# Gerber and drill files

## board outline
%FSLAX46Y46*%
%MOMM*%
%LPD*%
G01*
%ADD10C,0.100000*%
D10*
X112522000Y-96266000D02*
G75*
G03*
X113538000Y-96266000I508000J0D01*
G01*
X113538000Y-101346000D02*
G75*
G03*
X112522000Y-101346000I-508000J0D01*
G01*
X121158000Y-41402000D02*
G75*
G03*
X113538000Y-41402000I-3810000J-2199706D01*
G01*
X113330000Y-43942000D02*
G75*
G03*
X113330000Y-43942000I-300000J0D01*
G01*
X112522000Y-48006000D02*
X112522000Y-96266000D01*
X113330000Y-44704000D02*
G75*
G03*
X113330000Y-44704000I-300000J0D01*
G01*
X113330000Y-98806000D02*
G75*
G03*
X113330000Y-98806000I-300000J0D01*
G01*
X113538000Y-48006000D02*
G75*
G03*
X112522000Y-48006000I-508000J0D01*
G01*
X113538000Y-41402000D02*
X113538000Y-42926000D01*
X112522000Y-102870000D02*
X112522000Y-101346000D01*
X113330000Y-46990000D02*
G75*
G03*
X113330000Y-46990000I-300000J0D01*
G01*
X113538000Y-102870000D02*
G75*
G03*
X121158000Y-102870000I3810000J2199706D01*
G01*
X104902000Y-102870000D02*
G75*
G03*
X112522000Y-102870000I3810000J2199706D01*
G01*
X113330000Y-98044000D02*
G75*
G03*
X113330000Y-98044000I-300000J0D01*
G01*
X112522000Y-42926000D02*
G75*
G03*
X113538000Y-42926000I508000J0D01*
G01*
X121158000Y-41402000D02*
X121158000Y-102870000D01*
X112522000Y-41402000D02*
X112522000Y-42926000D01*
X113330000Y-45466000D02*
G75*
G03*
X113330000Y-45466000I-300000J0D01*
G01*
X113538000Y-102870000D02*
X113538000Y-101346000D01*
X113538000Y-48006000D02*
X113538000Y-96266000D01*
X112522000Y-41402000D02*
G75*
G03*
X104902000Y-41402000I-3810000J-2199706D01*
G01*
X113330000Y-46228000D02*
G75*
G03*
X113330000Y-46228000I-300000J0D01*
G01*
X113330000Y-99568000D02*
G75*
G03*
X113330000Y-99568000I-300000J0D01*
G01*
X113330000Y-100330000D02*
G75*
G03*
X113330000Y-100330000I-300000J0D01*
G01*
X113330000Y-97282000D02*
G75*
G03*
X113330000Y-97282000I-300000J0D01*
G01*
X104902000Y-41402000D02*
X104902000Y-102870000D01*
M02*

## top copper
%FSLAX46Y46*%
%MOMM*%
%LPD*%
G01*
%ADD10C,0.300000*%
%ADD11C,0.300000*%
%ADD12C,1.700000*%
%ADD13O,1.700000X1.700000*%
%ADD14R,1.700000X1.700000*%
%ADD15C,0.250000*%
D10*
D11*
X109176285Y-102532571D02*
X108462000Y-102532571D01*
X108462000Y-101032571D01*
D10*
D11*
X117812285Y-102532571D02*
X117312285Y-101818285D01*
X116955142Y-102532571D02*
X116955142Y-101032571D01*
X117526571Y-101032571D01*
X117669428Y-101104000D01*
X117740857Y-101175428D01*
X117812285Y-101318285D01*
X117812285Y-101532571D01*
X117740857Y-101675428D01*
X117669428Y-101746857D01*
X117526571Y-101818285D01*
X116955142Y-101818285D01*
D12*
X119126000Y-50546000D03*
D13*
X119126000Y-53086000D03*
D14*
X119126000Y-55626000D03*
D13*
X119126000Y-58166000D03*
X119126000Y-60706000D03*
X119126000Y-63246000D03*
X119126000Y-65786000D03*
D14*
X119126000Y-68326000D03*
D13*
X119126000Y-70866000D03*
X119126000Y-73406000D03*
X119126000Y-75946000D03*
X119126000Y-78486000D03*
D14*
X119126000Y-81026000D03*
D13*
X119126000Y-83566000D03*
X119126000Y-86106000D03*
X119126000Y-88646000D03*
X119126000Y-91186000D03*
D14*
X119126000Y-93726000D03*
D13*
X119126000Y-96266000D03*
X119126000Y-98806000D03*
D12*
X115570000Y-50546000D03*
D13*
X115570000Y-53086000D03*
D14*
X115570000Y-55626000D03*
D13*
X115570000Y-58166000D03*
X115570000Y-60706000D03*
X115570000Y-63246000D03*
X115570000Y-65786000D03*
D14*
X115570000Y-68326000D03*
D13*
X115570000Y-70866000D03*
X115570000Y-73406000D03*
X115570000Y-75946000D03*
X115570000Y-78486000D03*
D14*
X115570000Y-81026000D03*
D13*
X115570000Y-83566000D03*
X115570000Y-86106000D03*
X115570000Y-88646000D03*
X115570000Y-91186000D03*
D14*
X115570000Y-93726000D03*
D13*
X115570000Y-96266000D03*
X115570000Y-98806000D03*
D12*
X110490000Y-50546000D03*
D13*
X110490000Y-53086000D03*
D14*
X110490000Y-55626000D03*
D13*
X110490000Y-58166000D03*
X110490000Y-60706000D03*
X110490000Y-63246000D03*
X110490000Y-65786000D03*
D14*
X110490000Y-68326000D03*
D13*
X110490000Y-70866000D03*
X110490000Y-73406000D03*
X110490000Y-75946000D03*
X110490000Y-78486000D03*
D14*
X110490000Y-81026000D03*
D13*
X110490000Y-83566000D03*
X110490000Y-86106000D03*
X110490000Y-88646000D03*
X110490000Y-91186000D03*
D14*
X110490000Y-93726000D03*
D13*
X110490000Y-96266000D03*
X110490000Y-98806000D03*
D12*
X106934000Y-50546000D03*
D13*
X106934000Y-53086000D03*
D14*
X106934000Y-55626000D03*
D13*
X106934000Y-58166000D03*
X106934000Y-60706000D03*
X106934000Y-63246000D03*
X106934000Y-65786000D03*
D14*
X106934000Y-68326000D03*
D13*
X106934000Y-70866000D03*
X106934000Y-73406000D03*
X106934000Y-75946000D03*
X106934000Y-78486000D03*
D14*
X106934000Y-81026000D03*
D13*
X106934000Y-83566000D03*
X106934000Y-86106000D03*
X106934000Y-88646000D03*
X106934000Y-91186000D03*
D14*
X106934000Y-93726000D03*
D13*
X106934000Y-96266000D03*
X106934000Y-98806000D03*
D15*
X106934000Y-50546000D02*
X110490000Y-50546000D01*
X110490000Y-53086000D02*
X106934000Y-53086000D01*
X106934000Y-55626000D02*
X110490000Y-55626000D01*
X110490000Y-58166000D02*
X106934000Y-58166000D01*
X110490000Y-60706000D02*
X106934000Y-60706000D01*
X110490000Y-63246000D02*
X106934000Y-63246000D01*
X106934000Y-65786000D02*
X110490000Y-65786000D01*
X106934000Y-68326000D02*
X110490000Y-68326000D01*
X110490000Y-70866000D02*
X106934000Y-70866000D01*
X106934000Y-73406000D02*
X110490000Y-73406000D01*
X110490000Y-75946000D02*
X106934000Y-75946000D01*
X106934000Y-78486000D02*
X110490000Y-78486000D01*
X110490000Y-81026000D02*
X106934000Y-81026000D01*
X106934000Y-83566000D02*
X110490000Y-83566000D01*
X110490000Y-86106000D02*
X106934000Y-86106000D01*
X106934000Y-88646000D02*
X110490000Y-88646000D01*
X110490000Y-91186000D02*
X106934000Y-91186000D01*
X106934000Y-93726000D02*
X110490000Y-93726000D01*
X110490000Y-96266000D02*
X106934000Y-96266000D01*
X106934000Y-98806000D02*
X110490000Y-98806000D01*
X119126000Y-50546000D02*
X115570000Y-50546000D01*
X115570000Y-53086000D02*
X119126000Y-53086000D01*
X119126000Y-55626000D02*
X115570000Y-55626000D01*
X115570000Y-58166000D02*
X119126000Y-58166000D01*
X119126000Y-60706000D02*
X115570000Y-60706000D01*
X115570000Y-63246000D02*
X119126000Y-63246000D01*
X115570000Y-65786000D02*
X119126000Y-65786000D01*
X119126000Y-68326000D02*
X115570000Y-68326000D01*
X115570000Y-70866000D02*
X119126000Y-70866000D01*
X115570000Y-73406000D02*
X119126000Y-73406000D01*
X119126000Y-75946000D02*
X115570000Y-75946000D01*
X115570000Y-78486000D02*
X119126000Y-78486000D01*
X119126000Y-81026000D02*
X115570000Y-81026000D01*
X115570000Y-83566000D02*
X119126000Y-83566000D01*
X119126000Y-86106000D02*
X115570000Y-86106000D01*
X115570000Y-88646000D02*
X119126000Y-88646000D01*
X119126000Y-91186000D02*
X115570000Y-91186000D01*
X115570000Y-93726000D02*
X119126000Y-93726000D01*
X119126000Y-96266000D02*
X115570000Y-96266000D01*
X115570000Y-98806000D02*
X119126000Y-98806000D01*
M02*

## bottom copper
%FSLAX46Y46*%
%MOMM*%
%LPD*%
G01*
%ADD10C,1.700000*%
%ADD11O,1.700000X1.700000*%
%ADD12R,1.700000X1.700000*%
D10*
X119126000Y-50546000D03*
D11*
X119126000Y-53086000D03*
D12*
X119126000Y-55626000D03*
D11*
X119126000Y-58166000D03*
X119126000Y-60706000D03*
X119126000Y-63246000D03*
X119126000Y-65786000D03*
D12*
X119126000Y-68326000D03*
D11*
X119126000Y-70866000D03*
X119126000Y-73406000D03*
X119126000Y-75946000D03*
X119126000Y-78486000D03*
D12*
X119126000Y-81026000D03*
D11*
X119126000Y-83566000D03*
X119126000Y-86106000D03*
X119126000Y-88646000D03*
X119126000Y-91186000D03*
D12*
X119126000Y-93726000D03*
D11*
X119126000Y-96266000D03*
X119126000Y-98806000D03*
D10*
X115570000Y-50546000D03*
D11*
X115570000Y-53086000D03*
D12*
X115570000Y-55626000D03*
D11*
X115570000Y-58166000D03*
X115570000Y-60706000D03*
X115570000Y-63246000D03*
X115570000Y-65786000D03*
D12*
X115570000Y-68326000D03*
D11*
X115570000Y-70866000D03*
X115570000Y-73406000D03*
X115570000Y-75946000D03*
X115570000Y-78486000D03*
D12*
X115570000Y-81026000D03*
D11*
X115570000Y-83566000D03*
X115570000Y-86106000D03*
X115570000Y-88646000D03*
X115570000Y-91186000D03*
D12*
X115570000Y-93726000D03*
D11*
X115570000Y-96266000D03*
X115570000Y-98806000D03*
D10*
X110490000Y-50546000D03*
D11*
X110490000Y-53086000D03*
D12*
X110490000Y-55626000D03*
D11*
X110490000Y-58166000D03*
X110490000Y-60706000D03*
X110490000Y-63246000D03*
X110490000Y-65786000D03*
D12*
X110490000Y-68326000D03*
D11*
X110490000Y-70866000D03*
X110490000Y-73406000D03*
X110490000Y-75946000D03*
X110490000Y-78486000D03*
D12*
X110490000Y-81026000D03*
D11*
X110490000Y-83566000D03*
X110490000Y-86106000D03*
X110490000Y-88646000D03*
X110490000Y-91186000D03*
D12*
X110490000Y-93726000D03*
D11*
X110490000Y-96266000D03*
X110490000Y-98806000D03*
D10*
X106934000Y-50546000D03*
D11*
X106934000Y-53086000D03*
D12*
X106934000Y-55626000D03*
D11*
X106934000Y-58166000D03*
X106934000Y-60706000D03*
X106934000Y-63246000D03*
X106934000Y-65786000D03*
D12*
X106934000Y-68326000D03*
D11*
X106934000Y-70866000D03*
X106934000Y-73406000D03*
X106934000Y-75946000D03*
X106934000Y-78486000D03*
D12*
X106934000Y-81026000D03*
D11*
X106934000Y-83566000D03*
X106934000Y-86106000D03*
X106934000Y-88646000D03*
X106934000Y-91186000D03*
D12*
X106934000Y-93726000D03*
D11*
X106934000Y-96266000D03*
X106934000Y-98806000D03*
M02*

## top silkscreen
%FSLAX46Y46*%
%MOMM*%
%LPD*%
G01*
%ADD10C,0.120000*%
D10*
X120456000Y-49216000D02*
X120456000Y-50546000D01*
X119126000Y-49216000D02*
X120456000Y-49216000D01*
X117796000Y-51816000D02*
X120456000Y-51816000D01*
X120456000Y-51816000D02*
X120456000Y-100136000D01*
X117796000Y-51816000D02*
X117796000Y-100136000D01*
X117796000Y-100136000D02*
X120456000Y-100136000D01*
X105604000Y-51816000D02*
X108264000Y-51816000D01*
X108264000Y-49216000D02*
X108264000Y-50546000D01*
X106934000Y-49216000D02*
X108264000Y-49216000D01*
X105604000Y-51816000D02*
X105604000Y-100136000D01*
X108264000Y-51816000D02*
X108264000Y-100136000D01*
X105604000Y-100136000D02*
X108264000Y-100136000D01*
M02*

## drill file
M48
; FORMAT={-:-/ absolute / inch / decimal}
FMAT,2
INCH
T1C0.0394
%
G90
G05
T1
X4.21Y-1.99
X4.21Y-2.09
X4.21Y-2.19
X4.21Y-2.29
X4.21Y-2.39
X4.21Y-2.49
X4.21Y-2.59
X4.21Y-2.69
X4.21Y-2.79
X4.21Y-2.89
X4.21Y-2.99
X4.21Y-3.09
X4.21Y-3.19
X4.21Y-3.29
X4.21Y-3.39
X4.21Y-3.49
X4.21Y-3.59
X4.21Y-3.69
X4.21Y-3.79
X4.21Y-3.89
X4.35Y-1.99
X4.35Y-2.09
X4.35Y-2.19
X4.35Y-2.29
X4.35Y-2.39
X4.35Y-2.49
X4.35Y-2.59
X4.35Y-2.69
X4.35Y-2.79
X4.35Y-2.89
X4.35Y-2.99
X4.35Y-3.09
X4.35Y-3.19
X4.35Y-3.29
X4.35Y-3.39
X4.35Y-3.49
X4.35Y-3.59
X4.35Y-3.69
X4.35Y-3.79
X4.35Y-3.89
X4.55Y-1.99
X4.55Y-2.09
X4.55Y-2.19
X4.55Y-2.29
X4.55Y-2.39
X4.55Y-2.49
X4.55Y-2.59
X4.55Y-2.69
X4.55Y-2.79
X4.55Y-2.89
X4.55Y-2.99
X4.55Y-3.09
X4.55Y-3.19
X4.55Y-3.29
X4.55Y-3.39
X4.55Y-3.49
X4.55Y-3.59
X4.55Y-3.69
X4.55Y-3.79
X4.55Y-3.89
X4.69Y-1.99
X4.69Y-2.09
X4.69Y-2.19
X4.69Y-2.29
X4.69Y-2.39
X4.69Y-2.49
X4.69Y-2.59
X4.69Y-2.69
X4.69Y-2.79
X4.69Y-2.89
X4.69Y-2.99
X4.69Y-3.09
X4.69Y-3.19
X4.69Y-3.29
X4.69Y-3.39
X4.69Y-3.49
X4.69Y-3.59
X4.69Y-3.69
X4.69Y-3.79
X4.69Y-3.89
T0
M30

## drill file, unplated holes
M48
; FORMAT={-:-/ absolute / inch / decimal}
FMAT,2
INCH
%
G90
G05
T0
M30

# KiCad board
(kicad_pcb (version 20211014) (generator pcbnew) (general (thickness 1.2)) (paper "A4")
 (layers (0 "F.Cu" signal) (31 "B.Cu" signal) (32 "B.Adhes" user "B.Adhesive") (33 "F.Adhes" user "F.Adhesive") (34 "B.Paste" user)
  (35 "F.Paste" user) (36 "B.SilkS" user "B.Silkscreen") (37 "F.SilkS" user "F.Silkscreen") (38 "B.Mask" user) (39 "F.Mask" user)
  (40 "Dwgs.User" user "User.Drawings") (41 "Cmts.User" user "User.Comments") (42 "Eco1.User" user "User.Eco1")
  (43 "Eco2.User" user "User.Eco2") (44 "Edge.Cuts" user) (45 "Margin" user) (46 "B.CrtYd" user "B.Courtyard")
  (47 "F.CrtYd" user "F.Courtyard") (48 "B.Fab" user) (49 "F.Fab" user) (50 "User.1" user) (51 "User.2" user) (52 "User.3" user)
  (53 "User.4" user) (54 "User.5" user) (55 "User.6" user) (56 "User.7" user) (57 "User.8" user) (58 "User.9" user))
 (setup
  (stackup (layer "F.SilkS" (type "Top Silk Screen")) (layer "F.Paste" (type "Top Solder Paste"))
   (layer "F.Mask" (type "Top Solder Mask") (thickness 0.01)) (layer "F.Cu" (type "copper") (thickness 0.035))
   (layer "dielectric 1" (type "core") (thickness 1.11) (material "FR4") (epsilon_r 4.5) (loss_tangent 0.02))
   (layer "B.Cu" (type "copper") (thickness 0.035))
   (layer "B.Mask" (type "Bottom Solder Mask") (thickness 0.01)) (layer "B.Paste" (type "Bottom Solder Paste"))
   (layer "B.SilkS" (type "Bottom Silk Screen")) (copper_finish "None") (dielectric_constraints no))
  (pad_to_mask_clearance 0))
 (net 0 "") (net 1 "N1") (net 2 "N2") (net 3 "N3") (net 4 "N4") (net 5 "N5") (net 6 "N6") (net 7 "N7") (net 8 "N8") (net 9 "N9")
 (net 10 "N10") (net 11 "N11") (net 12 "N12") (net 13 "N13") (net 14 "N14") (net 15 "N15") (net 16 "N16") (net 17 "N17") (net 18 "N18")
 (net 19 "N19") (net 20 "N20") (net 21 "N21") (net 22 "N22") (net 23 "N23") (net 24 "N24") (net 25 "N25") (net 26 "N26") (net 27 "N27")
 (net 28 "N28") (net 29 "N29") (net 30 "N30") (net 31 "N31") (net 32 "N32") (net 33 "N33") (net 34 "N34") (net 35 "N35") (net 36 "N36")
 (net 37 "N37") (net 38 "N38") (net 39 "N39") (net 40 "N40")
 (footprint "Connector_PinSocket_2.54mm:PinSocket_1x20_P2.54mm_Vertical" (layer "F.Cu") (at 119.126 50.546)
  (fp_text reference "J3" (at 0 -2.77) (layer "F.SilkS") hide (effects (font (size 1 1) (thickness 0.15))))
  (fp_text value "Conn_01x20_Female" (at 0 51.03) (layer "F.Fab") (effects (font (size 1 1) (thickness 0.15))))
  (fp_line (start 1.33 -1.33) (end 1.33 0) (layer "F.SilkS") (width 0.12))
  (fp_line (start 0 -1.33) (end 1.33 -1.33) (layer "F.SilkS") (width 0.12))
  (fp_line (start -1.33 1.27) (end 1.33 1.27) (layer "F.SilkS") (width 0.12))
  (fp_line (start 1.33 1.27) (end 1.33 49.59) (layer "F.SilkS") (width 0.12))
  (fp_line (start -1.33 1.27) (end -1.33 49.59) (layer "F.SilkS") (width 0.12))
  (fp_line (start -1.33 49.59) (end 1.33 49.59) (layer "F.SilkS") (width 0.12))
  (pad "1" thru_hole circle (at 0 0) (size 1.7 1.7) (drill 1) (layers *.Cu *.Mask) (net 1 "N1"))
  (pad "2" thru_hole oval (at 0 2.54) (size 1.7 1.7) (drill 1) (layers *.Cu *.Mask) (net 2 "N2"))
  (pad "3" thru_hole rect (at 0 5.08) (size 1.7 1.7) (drill 1) (layers *.Cu *.Mask) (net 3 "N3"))
  (pad "4" thru_hole oval (at 0 7.62) (size 1.7 1.7) (drill 1) (layers *.Cu *.Mask) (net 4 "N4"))
  (pad "5" thru_hole oval (at 0 10.16) (size 1.7 1.7) (drill 1) (layers *.Cu *.Mask) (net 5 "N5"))
  (pad "6" thru_hole oval (at 0 12.7) (size 1.7 1.7) (drill 1) (layers *.Cu *.Mask) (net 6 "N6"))
  (pad "7" thru_hole oval (at 0 15.24) (size 1.7 1.7) (drill 1) (layers *.Cu *.Mask) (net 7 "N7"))
  (pad "8" thru_hole rect (at 0 17.78) (size 1.7 1.7) (drill 1) (layers *.Cu *.Mask) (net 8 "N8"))
  (pad "9" thru_hole oval (at 0 20.32) (size 1.7 1.7) (drill 1) (layers *.Cu *.Mask) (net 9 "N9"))
  (pad "10" thru_hole oval (at 0 22.86) (size 1.7 1.7) (drill 1) (layers *.Cu *.Mask) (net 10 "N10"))
  (pad "11" thru_hole oval (at 0 25.4) (size 1.7 1.7) (drill 1) (layers *.Cu *.Mask) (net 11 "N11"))
  (pad "12" thru_hole oval (at 0 27.94) (size 1.7 1.7) (drill 1) (layers *.Cu *.Mask) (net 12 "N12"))
  (pad "13" thru_hole rect (at 0 30.48) (size 1.7 1.7) (drill 1) (layers *.Cu *.Mask) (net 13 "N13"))
  (pad "14" thru_hole oval (at 0 33.02) (size 1.7 1.7) (drill 1) (layers *.Cu *.Mask) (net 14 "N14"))
  (pad "15" thru_hole oval (at 0 35.56) (size 1.7 1.7) (drill 1) (layers *.Cu *.Mask) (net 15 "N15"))
  (pad "16" thru_hole oval (at 0 38.1) (size 1.7 1.7) (drill 1) (layers *.Cu *.Mask) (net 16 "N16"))
  (pad "17" thru_hole oval (at 0 40.64) (size 1.7 1.7) (drill 1) (layers *.Cu *.Mask) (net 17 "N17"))
  (pad "18" thru_hole rect (at 0 43.18) (size 1.7 1.7) (drill 1) (layers *.Cu *.Mask) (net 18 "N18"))
  (pad "19" thru_hole oval (at 0 45.72) (size 1.7 1.7) (drill 1) (layers *.Cu *.Mask) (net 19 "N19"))
  (pad "20" thru_hole oval (at 0 48.26) (size 1.7 1.7) (drill 1) (layers *.Cu *.Mask) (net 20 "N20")))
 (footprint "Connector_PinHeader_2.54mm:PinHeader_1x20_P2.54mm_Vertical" (layer "F.Cu") (at 115.57 50.546)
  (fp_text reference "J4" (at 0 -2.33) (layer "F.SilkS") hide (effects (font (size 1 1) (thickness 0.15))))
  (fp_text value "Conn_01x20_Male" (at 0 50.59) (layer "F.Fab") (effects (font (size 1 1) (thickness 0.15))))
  (pad "1" thru_hole circle (at 0 0) (size 1.7 1.7) (drill 1) (layers *.Cu *.Mask) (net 1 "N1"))
  (pad "2" thru_hole oval (at 0 2.54) (size 1.7 1.7) (drill 1) (layers *.Cu *.Mask) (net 2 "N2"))
  (pad "3" thru_hole rect (at 0 5.08) (size 1.7 1.7) (drill 1) (layers *.Cu *.Mask) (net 3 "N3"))
  (pad "4" thru_hole oval (at 0 7.62) (size 1.7 1.7) (drill 1) (layers *.Cu *.Mask) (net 4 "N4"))
  (pad "5" thru_hole oval (at 0 10.16) (size 1.7 1.7) (drill 1) (layers *.Cu *.Mask) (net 5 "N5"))
  (pad "6" thru_hole oval (at 0 12.7) (size 1.7 1.7) (drill 1) (layers *.Cu *.Mask) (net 6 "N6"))
  (pad "7" thru_hole oval (at 0 15.24) (size 1.7 1.7) (drill 1) (layers *.Cu *.Mask) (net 7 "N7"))
  (pad "8" thru_hole rect (at 0 17.78) (size 1.7 1.7) (drill 1) (layers *.Cu *.Mask) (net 8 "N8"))
  (pad "9" thru_hole oval (at 0 20.32) (size 1.7 1.7) (drill 1) (layers *.Cu *.Mask) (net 9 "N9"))
  (pad "10" thru_hole oval (at 0 22.86) (size 1.7 1.7) (drill 1) (layers *.Cu *.Mask) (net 10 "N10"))
  (pad "11" thru_hole oval (at 0 25.4) (size 1.7 1.7) (drill 1) (layers *.Cu *.Mask) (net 11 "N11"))
  (pad "12" thru_hole oval (at 0 27.94) (size 1.7 1.7) (drill 1) (layers *.Cu *.Mask) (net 12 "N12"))
  (pad "13" thru_hole rect (at 0 30.48) (size 1.7 1.7) (drill 1) (layers *.Cu *.Mask) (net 13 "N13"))
  (pad "14" thru_hole oval (at 0 33.02) (size 1.7 1.7) (drill 1) (layers *.Cu *.Mask) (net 14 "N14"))
  (pad "15" thru_hole oval (at 0 35.56) (size 1.7 1.7) (drill 1) (layers *.Cu *.Mask) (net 15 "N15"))
  (pad "16" thru_hole oval (at 0 38.1) (size 1.7 1.7) (drill 1) (layers *.Cu *.Mask) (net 16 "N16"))
  (pad "17" thru_hole oval (at 0 40.64) (size 1.7 1.7) (drill 1) (layers *.Cu *.Mask) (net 17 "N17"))
  (pad "18" thru_hole rect (at 0 43.18) (size 1.7 1.7) (drill 1) (layers *.Cu *.Mask) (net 18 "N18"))
  (pad "19" thru_hole oval (at 0 45.72) (size 1.7 1.7) (drill 1) (layers *.Cu *.Mask) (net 19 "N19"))
  (pad "20" thru_hole oval (at 0 48.26) (size 1.7 1.7) (drill 1) (layers *.Cu *.Mask) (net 20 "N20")))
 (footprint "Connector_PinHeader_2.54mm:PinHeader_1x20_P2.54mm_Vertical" (layer "F.Cu") (at 110.49 50.546)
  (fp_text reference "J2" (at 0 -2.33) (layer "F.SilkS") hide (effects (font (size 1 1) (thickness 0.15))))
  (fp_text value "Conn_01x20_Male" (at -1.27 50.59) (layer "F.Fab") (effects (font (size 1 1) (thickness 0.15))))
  (pad "1" thru_hole circle (at 0 0) (size 1.7 1.7) (drill 1) (layers *.Cu *.Mask) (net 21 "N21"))
  (pad "2" thru_hole oval (at 0 2.54) (size 1.7 1.7) (drill 1) (layers *.Cu *.Mask) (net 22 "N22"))
  (pad "3" thru_hole rect (at 0 5.08) (size 1.7 1.7) (drill 1) (layers *.Cu *.Mask) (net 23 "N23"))
  (pad "4" thru_hole oval (at 0 7.62) (size 1.7 1.7) (drill 1) (layers *.Cu *.Mask) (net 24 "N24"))
  (pad "5" thru_hole oval (at 0 10.16) (size 1.7 1.7) (drill 1) (layers *.Cu *.Mask) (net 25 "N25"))
  (pad "6" thru_hole oval (at 0 12.7) (size 1.7 1.7) (drill 1) (layers *.Cu *.Mask) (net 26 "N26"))
  (pad "7" thru_hole oval (at 0 15.24) (size 1.7 1.7) (drill 1) (layers *.Cu *.Mask) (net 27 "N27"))
  (pad "8" thru_hole rect (at 0 17.78) (size 1.7 1.7) (drill 1) (layers *.Cu *.Mask) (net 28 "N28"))
  (pad "9" thru_hole oval (at 0 20.32) (size 1.7 1.7) (drill 1) (layers *.Cu *.Mask) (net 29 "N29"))
  (pad "10" thru_hole oval (at 0 22.86) (size 1.7 1.7) (drill 1) (layers *.Cu *.Mask) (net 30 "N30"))
  (pad "11" thru_hole oval (at 0 25.4) (size 1.7 1.7) (drill 1) (layers *.Cu *.Mask) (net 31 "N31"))
  (pad "12" thru_hole oval (at 0 27.94) (size 1.7 1.7) (drill 1) (layers *.Cu *.Mask) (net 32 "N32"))
  (pad "13" thru_hole rect (at 0 30.48) (size 1.7 1.7) (drill 1) (layers *.Cu *.Mask) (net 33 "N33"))
  (pad "14" thru_hole oval (at 0 33.02) (size 1.7 1.7) (drill 1) (layers *.Cu *.Mask) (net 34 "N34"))
  (pad "15" thru_hole oval (at 0 35.56) (size 1.7 1.7) (drill 1) (layers *.Cu *.Mask) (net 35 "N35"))
  (pad "16" thru_hole oval (at 0 38.1) (size 1.7 1.7) (drill 1) (layers *.Cu *.Mask) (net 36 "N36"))
  (pad "17" thru_hole oval (at 0 40.64) (size 1.7 1.7) (drill 1) (layers *.Cu *.Mask) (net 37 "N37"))
  (pad "18" thru_hole rect (at 0 43.18) (size 1.7 1.7) (drill 1) (layers *.Cu *.Mask) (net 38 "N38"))
  (pad "19" thru_hole oval (at 0 45.72) (size 1.7 1.7) (drill 1) (layers *.Cu *.Mask) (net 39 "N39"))
  (pad "20" thru_hole oval (at 0 48.26) (size 1.7 1.7) (drill 1) (layers *.Cu *.Mask) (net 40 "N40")))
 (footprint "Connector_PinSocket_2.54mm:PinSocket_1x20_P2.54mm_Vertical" (layer "F.Cu") (at 106.934 50.546)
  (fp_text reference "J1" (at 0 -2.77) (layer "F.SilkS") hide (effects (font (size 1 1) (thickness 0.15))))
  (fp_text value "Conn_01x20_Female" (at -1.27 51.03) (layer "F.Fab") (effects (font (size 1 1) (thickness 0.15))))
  (fp_line (start -1.33 1.27) (end 1.33 1.27) (layer "F.SilkS") (width 0.12))
  (fp_line (start 1.33 -1.33) (end 1.33 0) (layer "F.SilkS") (width 0.12))
  (fp_line (start 0 -1.33) (end 1.33 -1.33) (layer "F.SilkS") (width 0.12))
  (fp_line (start -1.33 1.27) (end -1.33 49.59) (layer "F.SilkS") (width 0.12))
  (fp_line (start 1.33 1.27) (end 1.33 49.59) (layer "F.SilkS") (width 0.12))
  (fp_line (start -1.33 49.59) (end 1.33 49.59) (layer "F.SilkS") (width 0.12))
  (pad "1" thru_hole circle (at 0 0) (size 1.7 1.7) (drill 1) (layers *.Cu *.Mask) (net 21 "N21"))
  (pad "2" thru_hole oval (at 0 2.54) (size 1.7 1.7) (drill 1) (layers *.Cu *.Mask) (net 22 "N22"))
  (pad "3" thru_hole rect (at 0 5.08) (size 1.7 1.7) (drill 1) (layers *.Cu *.Mask) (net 23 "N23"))
  (pad "4" thru_hole oval (at 0 7.62) (size 1.7 1.7) (drill 1) (layers *.Cu *.Mask) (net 24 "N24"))
  (pad "5" thru_hole oval (at 0 10.16) (size 1.7 1.7) (drill 1) (layers *.Cu *.Mask) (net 25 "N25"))
  (pad "6" thru_hole oval (at 0 12.7) (size 1.7 1.7) (drill 1) (layers *.Cu *.Mask) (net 26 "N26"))
  (pad "7" thru_hole oval (at 0 15.24) (size 1.7 1.7) (drill 1) (layers *.Cu *.Mask) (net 27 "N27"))
  (pad "8" thru_hole rect (at 0 17.78) (size 1.7 1.7) (drill 1) (layers *.Cu *.Mask) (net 28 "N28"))
  (pad "9" thru_hole oval (at 0 20.32) (size 1.7 1.7) (drill 1) (layers *.Cu *.Mask) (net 29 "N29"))
  (pad "10" thru_hole oval (at 0 22.86) (size 1.7 1.7) (drill 1) (layers *.Cu *.Mask) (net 30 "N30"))
  (pad "11" thru_hole oval (at 0 25.4) (size 1.7 1.7) (drill 1) (layers *.Cu *.Mask) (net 31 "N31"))
  (pad "12" thru_hole oval (at 0 27.94) (size 1.7 1.7) (drill 1) (layers *.Cu *.Mask) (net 32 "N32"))
  (pad "13" thru_hole rect (at 0 30.48) (size 1.7 1.7) (drill 1) (layers *.Cu *.Mask) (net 33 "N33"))
  (pad "14" thru_hole oval (at 0 33.02) (size 1.7 1.7) (drill 1) (layers *.Cu *.Mask) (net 34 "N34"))
  (pad "15" thru_hole oval (at 0 35.56) (size 1.7 1.7) (drill 1) (layers *.Cu *.Mask) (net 35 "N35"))
  (pad "16" thru_hole oval (at 0 38.1) (size 1.7 1.7) (drill 1) (layers *.Cu *.Mask) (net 36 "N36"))
  (pad "17" thru_hole oval (at 0 40.64) (size 1.7 1.7) (drill 1) (layers *.Cu *.Mask) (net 37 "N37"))
  (pad "18" thru_hole rect (at 0 43.18) (size 1.7 1.7) (drill 1) (layers *.Cu *.Mask) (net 38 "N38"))
  (pad "19" thru_hole oval (at 0 45.72) (size 1.7 1.7) (drill 1) (layers *.Cu *.Mask) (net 39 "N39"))
  (pad "20" thru_hole oval (at 0 48.26) (size 1.7 1.7) (drill 1) (layers *.Cu *.Mask) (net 40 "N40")))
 (gr_arc (start 113.538 96.266) (mid 113.03 96.774) (end 112.522 96.266) (layer "Edge.Cuts") (width 0.1))
 (gr_arc (start 112.522 101.346) (mid 113.03 100.838) (end 113.538 101.346) (layer "Edge.Cuts") (width 0.1))
 (gr_arc (start 113.538 41.402) (mid 117.348 39.202296) (end 121.158 41.402) (layer "Edge.Cuts") (width 0.1))
 (gr_circle (center 113.03 43.942) (end 113.33 43.942) (layer "Edge.Cuts") (width 0.1) (fill none))
 (gr_line (start 112.522 48.006) (end 112.522 96.266) (layer "Edge.Cuts") (width 0.1))
 (gr_circle (center 113.03 44.704) (end 113.33 44.704) (layer "Edge.Cuts") (width 0.1) (fill none))
 (gr_circle (center 113.03 98.806) (end 113.33 98.806) (layer "Edge.Cuts") (width 0.1) (fill none))
 (gr_arc (start 112.522 48.006) (mid 113.03 47.498) (end 113.538 48.006) (layer "Edge.Cuts") (width 0.1))
 (gr_line (start 113.538 41.402) (end 113.538 42.926) (layer "Edge.Cuts") (width 0.1))
 (gr_line (start 112.522 102.87) (end 112.522 101.346) (layer "Edge.Cuts") (width 0.1))
 (gr_circle (center 113.03 46.99) (end 113.33 46.99) (layer "Edge.Cuts") (width 0.1) (fill none))
 (gr_arc (start 121.158 102.87) (mid 117.348 105.069704) (end 113.538 102.87) (layer "Edge.Cuts") (width 0.1))
 (gr_arc (start 112.522 102.87) (mid 108.712 105.069704) (end 104.902 102.87) (layer "Edge.Cuts") (width 0.1))
 (gr_circle (center 113.03 98.044) (end 113.33 98.044) (layer "Edge.Cuts") (width 0.1) (fill none))
 (gr_arc (start 113.538 42.926) (mid 113.03 43.434) (end 112.522 42.926) (layer "Edge.Cuts") (width 0.1))
 (gr_line (start 121.158 41.402) (end 121.158 102.87) (layer "Edge.Cuts") (width 0.1))
 (gr_line (start 112.522 41.402) (end 112.522 42.926) (layer "Edge.Cuts") (width 0.1))
 (gr_circle (center 113.03 45.466) (end 113.33 45.466) (layer "Edge.Cuts") (width 0.1) (fill none))
 (gr_line (start 113.538 102.87) (end 113.538 101.346) (layer "Edge.Cuts") (width 0.1))
 (gr_line (start 113.538 48.006) (end 113.538 96.266) (layer "Edge.Cuts") (width 0.1))
 (gr_arc (start 104.902 41.402) (mid 108.712 39.202296) (end 112.522 41.402) (layer "Edge.Cuts") (width 0.1))
 (gr_circle (center 113.03 46.228) (end 113.33 46.228) (layer "Edge.Cuts") (width 0.1) (fill none))
 (gr_circle (center 113.03 99.568) (end 113.33 99.568) (layer "Edge.Cuts") (width 0.1) (fill none))
 (gr_circle (center 113.03 100.33) (end 113.33 100.33) (layer "Edge.Cuts") (width 0.1) (fill none))
 (gr_circle (center 113.03 97.282) (end 113.33 97.282) (layer "Edge.Cuts") (width 0.1) (fill none))
 (gr_line (start 104.902 41.402) (end 104.902 102.87) (layer "Edge.Cuts") (width 0.1))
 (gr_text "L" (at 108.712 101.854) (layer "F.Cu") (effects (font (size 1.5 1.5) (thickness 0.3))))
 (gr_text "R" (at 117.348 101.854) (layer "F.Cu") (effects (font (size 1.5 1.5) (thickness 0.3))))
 (segment (start 106.934 50.546) (end 110.49 50.546) (width 0.25) (layer "F.Cu") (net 21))
 (segment (start 110.49 53.086) (end 106.934 53.086) (width 0.25) (layer "F.Cu") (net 22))
 (segment (start 106.934 55.626) (end 110.49 55.626) (width 0.25) (layer "F.Cu") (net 23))
 (segment (start 110.49 58.166) (end 106.934 58.166) (width 0.25) (layer "F.Cu") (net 24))
 (segment (start 110.49 60.706) (end 106.934 60.706) (width 0.25) (layer "F.Cu") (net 25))
 (segment (start 110.49 63.246) (end 106.934 63.246) (width 0.25) (layer "F.Cu") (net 26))
 (segment (start 106.934 65.786) (end 110.49 65.786) (width 0.25) (layer "F.Cu") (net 27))
 (segment (start 106.934 68.326) (end 110.49 68.326) (width 0.25) (layer "F.Cu") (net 28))
 (segment (start 110.49 70.866) (end 106.934 70.866) (width 0.25) (layer "F.Cu") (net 29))
 (segment (start 106.934 73.406) (end 110.49 73.406) (width 0.25) (layer "F.Cu") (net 30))
 (segment (start 110.49 75.946) (end 106.934 75.946) (width 0.25) (layer "F.Cu") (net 31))
 (segment (start 106.934 78.486) (end 110.49 78.486) (width 0.25) (layer "F.Cu") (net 32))
 (segment (start 110.49 81.026) (end 106.934 81.026) (width 0.25) (layer "F.Cu") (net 33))
 (segment (start 106.934 83.566) (end 110.49 83.566) (width 0.25) (layer "F.Cu") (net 34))
 (segment (start 110.49 86.106) (end 106.934 86.106) (width 0.25) (layer "F.Cu") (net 35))
 (segment (start 106.934 88.646) (end 110.49 88.646) (width 0.25) (layer "F.Cu") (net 36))
 (segment (start 110.49 91.186) (end 106.934 91.186) (width 0.25) (layer "F.Cu") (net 37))
 (segment (start 106.934 93.726) (end 110.49 93.726) (width 0.25) (layer "F.Cu") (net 38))
 (segment (start 110.49 96.266) (end 106.934 96.266) (width 0.25) (layer "F.Cu") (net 39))
 (segment (start 106.934 98.806) (end 110.49 98.806) (width 0.25) (layer "F.Cu") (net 40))
 (segment (start 119.126 50.546) (end 115.57 50.546) (width 0.25) (layer "F.Cu") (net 1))
 (segment (start 115.57 53.086) (end 119.126 53.086) (width 0.25) (layer "F.Cu") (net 2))
 (segment (start 119.126 55.626) (end 115.57 55.626) (width 0.25) (layer "F.Cu") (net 3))
 (segment (start 115.57 58.166) (end 119.126 58.166) (width 0.25) (layer "F.Cu") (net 4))
 (segment (start 119.126 60.706) (end 115.57 60.706) (width 0.25) (layer "F.Cu") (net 5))
 (segment (start 115.57 63.246) (end 119.126 63.246) (width 0.25) (layer "F.Cu") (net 6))
 (segment (start 115.57 65.786) (end 119.126 65.786) (width 0.25) (layer "F.Cu") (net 7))
 (segment (start 119.126 68.326) (end 115.57 68.326) (width 0.25) (layer "F.Cu") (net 8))
 (segment (start 115.57 70.866) (end 119.126 70.866) (width 0.25) (layer "F.Cu") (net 9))
 (segment (start 115.57 73.406) (end 119.126 73.406) (width 0.25) (layer "F.Cu") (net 10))
 (segment (start 119.126 75.946) (end 115.57 75.946) (width 0.25) (layer "F.Cu") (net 11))
 (segment (start 115.57 78.486) (end 119.126 78.486) (width 0.25) (layer "F.Cu") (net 12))
 (segment (start 119.126 81.026) (end 115.57 81.026) (width 0.25) (layer "F.Cu") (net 13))
 (segment (start 115.57 83.566) (end 119.126 83.566) (width 0.25) (layer "F.Cu") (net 14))
 (segment (start 119.126 86.106) (end 115.57 86.106) (width 0.25) (layer "F.Cu") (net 15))
 (segment (start 115.57 88.646) (end 119.126 88.646) (width 0.25) (layer "F.Cu") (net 16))
 (segment (start 119.126 91.186) (end 115.57 91.186) (width 0.25) (layer "F.Cu") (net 17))
 (segment (start 115.57 93.726) (end 119.126 93.726) (width 0.25) (layer "F.Cu") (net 18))
 (segment (start 119.126 96.266) (end 115.57 96.266) (width 0.25) (layer "F.Cu") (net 19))
 (segment (start 115.57 98.806) (end 119.126 98.806) (width 0.25) (layer "F.Cu") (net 20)))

